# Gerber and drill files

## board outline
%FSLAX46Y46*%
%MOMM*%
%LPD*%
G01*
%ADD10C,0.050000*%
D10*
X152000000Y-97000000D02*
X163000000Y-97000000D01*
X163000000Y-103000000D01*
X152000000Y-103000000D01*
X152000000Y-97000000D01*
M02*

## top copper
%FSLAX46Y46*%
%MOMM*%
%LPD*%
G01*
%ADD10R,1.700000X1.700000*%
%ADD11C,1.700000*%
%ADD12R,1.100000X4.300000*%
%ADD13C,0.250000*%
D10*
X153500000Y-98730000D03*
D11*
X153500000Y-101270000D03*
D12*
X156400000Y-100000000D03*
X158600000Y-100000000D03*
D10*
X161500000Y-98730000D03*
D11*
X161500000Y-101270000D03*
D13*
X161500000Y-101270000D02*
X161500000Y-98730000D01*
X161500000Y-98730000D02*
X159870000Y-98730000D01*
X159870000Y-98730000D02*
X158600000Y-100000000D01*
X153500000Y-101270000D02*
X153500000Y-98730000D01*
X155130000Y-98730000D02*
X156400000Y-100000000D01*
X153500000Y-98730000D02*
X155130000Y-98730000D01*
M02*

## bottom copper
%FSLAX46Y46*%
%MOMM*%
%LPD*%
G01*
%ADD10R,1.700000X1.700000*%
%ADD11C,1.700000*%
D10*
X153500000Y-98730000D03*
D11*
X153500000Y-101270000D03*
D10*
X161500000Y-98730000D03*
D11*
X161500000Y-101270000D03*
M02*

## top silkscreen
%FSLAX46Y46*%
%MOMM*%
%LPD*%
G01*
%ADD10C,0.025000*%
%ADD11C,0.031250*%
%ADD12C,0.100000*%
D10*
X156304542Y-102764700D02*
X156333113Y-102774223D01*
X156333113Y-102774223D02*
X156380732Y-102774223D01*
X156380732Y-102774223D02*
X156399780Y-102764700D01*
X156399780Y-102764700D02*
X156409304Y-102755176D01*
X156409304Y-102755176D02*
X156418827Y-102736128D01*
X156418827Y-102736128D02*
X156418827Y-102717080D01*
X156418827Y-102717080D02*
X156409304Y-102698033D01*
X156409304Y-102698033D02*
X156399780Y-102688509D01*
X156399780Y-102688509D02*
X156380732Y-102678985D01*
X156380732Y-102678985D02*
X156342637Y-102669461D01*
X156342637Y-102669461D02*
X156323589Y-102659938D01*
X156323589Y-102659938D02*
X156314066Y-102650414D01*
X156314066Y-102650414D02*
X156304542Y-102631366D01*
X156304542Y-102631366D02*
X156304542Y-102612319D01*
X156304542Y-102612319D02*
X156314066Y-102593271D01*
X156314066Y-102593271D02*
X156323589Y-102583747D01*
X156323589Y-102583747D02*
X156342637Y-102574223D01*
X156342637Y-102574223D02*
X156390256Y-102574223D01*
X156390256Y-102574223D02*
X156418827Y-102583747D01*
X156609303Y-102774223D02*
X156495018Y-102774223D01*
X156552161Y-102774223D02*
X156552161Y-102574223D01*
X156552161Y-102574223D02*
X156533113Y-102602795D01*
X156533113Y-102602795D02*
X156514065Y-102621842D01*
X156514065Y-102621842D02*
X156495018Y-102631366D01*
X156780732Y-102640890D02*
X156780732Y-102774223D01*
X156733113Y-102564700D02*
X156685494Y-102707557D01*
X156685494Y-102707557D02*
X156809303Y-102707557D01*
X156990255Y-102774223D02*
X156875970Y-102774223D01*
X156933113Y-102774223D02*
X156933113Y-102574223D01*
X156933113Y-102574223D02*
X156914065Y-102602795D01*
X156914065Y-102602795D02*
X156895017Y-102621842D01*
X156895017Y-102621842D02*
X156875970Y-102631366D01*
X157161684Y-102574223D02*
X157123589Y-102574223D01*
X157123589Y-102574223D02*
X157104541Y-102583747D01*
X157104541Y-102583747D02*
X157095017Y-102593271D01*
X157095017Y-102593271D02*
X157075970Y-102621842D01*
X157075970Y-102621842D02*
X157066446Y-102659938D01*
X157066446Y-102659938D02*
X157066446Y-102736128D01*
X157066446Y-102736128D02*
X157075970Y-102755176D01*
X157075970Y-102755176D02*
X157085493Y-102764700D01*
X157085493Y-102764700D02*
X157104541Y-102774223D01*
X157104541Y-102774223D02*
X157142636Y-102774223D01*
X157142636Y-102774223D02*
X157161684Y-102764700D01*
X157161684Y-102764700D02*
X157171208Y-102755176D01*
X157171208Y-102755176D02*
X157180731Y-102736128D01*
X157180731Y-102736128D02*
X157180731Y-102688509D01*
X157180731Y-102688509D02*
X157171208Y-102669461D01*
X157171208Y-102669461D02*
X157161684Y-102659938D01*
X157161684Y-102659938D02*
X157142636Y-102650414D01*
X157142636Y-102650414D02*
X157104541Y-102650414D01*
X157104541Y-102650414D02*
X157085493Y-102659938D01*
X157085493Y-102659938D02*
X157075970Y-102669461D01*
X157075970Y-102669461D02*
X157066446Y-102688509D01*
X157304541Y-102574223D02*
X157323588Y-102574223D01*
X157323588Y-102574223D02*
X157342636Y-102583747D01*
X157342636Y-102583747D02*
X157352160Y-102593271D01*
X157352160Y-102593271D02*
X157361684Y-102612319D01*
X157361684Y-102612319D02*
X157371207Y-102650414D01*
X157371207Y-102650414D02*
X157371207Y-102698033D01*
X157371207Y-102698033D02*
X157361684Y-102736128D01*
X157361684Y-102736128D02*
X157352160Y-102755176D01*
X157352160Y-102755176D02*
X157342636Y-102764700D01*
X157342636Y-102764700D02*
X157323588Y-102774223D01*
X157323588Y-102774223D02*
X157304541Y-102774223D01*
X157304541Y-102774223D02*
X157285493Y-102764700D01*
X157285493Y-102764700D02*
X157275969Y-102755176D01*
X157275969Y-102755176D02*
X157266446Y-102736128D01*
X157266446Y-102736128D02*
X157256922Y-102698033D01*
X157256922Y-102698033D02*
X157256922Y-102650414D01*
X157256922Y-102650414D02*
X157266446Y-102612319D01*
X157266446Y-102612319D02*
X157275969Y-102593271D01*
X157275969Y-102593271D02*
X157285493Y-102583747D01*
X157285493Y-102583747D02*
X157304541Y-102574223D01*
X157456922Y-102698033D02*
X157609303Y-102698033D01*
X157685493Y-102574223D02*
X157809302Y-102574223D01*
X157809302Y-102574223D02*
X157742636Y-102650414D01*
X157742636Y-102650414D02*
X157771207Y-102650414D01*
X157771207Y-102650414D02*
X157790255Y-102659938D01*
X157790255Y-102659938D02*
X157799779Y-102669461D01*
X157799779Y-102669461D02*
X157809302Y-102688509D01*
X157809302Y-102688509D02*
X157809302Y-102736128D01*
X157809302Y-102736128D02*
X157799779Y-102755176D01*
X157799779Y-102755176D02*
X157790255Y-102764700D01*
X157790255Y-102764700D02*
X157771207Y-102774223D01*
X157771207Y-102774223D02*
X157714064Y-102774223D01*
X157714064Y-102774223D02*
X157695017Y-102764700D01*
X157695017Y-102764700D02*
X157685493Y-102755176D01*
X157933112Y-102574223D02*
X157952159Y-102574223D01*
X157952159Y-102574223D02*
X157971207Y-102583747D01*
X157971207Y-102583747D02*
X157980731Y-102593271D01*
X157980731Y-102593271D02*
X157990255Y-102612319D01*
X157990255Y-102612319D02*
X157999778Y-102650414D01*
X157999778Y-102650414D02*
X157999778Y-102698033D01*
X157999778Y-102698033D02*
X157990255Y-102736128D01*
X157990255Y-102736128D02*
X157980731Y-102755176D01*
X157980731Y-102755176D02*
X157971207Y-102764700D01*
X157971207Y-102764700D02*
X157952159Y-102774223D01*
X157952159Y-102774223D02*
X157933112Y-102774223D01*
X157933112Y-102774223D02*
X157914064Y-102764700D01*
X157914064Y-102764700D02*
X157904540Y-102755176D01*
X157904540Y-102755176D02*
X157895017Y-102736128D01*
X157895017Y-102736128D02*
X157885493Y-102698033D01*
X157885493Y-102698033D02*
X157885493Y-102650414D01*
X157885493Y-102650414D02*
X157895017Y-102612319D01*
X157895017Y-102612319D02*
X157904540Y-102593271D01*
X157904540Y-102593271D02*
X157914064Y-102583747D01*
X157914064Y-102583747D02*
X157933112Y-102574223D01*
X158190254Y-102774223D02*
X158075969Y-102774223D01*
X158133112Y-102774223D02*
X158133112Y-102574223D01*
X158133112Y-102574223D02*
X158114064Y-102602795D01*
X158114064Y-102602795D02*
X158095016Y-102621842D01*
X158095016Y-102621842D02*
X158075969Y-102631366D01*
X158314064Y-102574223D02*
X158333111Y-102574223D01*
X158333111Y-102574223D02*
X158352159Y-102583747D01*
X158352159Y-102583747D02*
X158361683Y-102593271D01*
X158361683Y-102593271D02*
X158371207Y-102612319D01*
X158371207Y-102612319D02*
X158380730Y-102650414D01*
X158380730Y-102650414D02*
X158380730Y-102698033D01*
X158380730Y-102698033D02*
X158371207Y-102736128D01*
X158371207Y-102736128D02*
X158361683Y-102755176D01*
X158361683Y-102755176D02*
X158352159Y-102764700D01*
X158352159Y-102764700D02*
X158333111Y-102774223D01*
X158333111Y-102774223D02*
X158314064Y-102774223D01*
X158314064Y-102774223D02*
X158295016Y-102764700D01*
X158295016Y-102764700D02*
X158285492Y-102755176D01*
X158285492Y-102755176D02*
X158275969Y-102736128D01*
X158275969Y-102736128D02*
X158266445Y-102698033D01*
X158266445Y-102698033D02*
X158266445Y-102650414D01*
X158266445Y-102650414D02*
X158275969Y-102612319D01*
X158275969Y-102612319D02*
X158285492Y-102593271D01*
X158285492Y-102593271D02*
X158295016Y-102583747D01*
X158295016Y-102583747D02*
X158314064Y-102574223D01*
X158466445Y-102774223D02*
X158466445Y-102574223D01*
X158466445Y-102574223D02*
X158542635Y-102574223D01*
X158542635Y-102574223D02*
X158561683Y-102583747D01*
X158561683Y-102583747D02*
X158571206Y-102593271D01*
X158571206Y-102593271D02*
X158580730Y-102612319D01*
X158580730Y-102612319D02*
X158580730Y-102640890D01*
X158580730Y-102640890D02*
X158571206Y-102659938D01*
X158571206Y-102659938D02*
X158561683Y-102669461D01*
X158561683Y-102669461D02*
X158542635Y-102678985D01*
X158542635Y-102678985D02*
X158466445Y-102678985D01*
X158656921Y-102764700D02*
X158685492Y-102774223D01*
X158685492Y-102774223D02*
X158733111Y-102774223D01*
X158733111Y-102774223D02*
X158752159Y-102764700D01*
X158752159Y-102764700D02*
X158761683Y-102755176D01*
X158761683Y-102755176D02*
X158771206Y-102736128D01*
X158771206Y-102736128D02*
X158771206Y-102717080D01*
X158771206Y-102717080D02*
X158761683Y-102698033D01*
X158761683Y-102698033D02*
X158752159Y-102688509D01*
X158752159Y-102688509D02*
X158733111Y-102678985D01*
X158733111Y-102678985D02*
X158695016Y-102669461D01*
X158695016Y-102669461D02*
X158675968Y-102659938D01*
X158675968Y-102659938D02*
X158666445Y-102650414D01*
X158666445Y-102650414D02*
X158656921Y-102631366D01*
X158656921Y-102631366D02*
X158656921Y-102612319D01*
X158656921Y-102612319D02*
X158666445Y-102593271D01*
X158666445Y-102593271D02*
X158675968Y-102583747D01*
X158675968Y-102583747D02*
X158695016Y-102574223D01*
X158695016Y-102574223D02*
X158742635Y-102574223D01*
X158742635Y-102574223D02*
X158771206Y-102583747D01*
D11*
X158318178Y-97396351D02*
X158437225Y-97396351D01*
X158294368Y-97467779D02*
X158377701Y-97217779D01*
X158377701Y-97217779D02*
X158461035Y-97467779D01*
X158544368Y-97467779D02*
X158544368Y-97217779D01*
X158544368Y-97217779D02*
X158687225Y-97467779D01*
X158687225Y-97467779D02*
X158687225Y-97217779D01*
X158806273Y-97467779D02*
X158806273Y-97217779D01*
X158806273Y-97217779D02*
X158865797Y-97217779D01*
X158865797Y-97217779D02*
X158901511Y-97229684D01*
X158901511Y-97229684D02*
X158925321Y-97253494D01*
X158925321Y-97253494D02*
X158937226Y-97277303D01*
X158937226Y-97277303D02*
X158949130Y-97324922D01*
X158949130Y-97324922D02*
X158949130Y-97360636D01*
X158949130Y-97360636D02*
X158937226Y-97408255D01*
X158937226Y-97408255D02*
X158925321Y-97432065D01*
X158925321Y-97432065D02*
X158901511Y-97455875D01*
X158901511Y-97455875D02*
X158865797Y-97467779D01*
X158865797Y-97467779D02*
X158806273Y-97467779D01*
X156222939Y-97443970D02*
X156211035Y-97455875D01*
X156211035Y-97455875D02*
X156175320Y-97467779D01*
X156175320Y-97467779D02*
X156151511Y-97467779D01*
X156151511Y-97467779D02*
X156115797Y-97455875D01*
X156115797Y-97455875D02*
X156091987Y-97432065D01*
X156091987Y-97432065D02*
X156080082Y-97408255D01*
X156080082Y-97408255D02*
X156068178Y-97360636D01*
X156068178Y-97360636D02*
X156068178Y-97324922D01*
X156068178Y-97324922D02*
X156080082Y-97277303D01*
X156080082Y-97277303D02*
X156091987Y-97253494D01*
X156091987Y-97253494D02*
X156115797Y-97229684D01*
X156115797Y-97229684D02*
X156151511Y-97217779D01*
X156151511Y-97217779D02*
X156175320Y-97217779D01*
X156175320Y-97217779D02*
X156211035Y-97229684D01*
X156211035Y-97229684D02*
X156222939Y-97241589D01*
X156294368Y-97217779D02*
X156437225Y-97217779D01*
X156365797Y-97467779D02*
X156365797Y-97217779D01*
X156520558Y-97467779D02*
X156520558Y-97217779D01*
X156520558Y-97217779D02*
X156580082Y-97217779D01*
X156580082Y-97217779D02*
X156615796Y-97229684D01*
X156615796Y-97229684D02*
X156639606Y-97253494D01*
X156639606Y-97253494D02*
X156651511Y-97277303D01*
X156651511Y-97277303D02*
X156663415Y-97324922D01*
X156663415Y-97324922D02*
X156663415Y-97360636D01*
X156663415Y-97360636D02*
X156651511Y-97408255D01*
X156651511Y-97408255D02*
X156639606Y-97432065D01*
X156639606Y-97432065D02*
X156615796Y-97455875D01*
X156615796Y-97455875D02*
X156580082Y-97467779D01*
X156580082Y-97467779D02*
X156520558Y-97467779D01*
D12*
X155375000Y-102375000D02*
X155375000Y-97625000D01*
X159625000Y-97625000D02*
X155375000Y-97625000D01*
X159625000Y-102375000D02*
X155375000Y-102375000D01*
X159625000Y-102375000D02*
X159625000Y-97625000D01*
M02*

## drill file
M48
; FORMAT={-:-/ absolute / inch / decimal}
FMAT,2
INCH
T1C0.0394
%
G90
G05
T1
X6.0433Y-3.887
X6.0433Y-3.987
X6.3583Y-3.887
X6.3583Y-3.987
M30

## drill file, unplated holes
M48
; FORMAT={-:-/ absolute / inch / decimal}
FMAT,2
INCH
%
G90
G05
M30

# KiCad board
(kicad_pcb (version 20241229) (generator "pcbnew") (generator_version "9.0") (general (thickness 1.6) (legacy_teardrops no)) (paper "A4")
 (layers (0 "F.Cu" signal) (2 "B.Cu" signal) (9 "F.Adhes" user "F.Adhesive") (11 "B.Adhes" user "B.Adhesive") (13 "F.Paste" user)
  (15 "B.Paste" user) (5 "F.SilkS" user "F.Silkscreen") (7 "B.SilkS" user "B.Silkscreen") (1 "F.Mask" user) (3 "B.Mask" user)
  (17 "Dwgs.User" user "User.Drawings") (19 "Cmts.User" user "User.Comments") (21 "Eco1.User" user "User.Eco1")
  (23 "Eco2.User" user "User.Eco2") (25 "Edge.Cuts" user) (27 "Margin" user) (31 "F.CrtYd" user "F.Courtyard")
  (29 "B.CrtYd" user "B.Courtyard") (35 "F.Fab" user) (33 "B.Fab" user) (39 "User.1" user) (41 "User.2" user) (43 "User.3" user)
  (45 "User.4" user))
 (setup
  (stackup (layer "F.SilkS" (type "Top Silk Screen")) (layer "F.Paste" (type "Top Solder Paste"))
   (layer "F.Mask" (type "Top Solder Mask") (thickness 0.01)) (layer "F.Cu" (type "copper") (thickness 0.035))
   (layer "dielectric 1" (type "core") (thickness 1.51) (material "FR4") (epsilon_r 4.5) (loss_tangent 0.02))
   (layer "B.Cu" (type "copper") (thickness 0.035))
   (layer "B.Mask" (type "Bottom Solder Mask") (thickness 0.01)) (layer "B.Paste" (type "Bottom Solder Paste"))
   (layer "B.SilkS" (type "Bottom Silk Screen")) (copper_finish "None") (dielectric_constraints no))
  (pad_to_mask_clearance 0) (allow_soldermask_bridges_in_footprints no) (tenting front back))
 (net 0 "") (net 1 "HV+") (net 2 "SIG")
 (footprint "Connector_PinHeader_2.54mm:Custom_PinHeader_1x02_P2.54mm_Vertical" (layer "F.Cu") (at 153.5 98.73)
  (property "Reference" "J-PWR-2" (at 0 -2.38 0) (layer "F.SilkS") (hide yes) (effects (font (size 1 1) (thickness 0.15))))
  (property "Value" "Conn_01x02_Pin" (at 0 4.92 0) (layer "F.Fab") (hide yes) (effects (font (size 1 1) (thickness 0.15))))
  (pad "1" thru_hole rect (at 0 0) (size 1.7 1.7) (drill 1) (layers "*.Cu" "*.Mask") (remove_unused_layers no) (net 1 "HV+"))
  (pad "2" thru_hole circle (at 0 2.54) (size 1.7 1.7) (drill 1) (layers "*.Cu" "*.Mask") (remove_unused_layers no) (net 1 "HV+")))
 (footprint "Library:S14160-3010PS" (layer "F.Cu") (at 157.5 100)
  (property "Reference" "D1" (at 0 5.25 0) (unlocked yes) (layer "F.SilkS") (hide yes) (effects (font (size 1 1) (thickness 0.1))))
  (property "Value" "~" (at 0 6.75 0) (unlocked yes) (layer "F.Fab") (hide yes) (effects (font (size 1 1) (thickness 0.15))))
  (fp_line (start -2.125 2.375) (end -2.125 -2.375) (stroke (width 0.1) (type default)) (layer "F.SilkS"))
  (fp_line (start 2.125 -2.375) (end -2.125 -2.375) (stroke (width 0.1) (type default)) (layer "F.SilkS"))
  (fp_line (start 2.125 2.375) (end -2.125 2.375) (stroke (width 0.1) (type default)) (layer "F.SilkS"))
  (fp_line (start 2.125 2.375) (end 2.125 -2.375) (stroke (width 0.1) (type default)) (layer "F.SilkS"))
  (pad "1" smd rect (at -1.1 0) (size 1.1 4.3) (layers "F.Cu" "F.Mask" "F.Paste") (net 1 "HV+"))
  (pad "2" smd rect (at 1.1 0) (size 1.1 4.3) (layers "F.Cu" "F.Mask" "F.Paste") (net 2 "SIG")))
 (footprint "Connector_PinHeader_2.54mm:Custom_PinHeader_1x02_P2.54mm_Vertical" (layer "F.Cu") (at 161.5 98.73)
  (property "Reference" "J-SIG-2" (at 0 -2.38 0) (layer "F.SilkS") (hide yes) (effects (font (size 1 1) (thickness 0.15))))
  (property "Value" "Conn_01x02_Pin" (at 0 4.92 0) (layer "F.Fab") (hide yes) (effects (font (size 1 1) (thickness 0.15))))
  (pad "1" thru_hole rect (at 0 0) (size 1.7 1.7) (drill 1) (layers "*.Cu" "*.Mask") (remove_unused_layers no) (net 2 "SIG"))
  (pad "2" thru_hole circle (at 0 2.54) (size 1.7 1.7) (drill 1) (layers "*.Cu" "*.Mask") (remove_unused_layers no) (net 2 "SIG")))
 (gr_rect (start 152 97) (end 163 103) (stroke (width 0.05) (type default)) (fill no) (layer "Edge.Cuts"))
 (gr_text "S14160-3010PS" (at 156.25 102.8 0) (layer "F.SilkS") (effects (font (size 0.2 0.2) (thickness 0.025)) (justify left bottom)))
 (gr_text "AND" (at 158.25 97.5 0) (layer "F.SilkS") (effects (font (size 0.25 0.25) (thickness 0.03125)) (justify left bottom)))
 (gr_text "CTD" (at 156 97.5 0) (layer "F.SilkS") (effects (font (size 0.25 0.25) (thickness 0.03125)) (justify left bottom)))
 (segment (start 161.5 101.27) (end 161.5 98.73) (width 0.25) (layer "F.Cu") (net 2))
 (segment (start 161.5 98.73) (end 159.87 98.73) (width 0.25) (layer "F.Cu") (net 2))
 (segment (start 159.87 98.73) (end 158.6 100) (width 0.25) (layer "F.Cu") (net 2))
 (segment (start 153.5 101.27) (end 153.5 98.73) (width 0.25) (layer "F.Cu") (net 1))
 (segment (start 155.13 98.73) (end 156.4 100) (width 0.25) (layer "F.Cu") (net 1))
 (segment (start 153.5 98.73) (end 155.13 98.73) (width 0.25) (layer "F.Cu") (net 1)))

